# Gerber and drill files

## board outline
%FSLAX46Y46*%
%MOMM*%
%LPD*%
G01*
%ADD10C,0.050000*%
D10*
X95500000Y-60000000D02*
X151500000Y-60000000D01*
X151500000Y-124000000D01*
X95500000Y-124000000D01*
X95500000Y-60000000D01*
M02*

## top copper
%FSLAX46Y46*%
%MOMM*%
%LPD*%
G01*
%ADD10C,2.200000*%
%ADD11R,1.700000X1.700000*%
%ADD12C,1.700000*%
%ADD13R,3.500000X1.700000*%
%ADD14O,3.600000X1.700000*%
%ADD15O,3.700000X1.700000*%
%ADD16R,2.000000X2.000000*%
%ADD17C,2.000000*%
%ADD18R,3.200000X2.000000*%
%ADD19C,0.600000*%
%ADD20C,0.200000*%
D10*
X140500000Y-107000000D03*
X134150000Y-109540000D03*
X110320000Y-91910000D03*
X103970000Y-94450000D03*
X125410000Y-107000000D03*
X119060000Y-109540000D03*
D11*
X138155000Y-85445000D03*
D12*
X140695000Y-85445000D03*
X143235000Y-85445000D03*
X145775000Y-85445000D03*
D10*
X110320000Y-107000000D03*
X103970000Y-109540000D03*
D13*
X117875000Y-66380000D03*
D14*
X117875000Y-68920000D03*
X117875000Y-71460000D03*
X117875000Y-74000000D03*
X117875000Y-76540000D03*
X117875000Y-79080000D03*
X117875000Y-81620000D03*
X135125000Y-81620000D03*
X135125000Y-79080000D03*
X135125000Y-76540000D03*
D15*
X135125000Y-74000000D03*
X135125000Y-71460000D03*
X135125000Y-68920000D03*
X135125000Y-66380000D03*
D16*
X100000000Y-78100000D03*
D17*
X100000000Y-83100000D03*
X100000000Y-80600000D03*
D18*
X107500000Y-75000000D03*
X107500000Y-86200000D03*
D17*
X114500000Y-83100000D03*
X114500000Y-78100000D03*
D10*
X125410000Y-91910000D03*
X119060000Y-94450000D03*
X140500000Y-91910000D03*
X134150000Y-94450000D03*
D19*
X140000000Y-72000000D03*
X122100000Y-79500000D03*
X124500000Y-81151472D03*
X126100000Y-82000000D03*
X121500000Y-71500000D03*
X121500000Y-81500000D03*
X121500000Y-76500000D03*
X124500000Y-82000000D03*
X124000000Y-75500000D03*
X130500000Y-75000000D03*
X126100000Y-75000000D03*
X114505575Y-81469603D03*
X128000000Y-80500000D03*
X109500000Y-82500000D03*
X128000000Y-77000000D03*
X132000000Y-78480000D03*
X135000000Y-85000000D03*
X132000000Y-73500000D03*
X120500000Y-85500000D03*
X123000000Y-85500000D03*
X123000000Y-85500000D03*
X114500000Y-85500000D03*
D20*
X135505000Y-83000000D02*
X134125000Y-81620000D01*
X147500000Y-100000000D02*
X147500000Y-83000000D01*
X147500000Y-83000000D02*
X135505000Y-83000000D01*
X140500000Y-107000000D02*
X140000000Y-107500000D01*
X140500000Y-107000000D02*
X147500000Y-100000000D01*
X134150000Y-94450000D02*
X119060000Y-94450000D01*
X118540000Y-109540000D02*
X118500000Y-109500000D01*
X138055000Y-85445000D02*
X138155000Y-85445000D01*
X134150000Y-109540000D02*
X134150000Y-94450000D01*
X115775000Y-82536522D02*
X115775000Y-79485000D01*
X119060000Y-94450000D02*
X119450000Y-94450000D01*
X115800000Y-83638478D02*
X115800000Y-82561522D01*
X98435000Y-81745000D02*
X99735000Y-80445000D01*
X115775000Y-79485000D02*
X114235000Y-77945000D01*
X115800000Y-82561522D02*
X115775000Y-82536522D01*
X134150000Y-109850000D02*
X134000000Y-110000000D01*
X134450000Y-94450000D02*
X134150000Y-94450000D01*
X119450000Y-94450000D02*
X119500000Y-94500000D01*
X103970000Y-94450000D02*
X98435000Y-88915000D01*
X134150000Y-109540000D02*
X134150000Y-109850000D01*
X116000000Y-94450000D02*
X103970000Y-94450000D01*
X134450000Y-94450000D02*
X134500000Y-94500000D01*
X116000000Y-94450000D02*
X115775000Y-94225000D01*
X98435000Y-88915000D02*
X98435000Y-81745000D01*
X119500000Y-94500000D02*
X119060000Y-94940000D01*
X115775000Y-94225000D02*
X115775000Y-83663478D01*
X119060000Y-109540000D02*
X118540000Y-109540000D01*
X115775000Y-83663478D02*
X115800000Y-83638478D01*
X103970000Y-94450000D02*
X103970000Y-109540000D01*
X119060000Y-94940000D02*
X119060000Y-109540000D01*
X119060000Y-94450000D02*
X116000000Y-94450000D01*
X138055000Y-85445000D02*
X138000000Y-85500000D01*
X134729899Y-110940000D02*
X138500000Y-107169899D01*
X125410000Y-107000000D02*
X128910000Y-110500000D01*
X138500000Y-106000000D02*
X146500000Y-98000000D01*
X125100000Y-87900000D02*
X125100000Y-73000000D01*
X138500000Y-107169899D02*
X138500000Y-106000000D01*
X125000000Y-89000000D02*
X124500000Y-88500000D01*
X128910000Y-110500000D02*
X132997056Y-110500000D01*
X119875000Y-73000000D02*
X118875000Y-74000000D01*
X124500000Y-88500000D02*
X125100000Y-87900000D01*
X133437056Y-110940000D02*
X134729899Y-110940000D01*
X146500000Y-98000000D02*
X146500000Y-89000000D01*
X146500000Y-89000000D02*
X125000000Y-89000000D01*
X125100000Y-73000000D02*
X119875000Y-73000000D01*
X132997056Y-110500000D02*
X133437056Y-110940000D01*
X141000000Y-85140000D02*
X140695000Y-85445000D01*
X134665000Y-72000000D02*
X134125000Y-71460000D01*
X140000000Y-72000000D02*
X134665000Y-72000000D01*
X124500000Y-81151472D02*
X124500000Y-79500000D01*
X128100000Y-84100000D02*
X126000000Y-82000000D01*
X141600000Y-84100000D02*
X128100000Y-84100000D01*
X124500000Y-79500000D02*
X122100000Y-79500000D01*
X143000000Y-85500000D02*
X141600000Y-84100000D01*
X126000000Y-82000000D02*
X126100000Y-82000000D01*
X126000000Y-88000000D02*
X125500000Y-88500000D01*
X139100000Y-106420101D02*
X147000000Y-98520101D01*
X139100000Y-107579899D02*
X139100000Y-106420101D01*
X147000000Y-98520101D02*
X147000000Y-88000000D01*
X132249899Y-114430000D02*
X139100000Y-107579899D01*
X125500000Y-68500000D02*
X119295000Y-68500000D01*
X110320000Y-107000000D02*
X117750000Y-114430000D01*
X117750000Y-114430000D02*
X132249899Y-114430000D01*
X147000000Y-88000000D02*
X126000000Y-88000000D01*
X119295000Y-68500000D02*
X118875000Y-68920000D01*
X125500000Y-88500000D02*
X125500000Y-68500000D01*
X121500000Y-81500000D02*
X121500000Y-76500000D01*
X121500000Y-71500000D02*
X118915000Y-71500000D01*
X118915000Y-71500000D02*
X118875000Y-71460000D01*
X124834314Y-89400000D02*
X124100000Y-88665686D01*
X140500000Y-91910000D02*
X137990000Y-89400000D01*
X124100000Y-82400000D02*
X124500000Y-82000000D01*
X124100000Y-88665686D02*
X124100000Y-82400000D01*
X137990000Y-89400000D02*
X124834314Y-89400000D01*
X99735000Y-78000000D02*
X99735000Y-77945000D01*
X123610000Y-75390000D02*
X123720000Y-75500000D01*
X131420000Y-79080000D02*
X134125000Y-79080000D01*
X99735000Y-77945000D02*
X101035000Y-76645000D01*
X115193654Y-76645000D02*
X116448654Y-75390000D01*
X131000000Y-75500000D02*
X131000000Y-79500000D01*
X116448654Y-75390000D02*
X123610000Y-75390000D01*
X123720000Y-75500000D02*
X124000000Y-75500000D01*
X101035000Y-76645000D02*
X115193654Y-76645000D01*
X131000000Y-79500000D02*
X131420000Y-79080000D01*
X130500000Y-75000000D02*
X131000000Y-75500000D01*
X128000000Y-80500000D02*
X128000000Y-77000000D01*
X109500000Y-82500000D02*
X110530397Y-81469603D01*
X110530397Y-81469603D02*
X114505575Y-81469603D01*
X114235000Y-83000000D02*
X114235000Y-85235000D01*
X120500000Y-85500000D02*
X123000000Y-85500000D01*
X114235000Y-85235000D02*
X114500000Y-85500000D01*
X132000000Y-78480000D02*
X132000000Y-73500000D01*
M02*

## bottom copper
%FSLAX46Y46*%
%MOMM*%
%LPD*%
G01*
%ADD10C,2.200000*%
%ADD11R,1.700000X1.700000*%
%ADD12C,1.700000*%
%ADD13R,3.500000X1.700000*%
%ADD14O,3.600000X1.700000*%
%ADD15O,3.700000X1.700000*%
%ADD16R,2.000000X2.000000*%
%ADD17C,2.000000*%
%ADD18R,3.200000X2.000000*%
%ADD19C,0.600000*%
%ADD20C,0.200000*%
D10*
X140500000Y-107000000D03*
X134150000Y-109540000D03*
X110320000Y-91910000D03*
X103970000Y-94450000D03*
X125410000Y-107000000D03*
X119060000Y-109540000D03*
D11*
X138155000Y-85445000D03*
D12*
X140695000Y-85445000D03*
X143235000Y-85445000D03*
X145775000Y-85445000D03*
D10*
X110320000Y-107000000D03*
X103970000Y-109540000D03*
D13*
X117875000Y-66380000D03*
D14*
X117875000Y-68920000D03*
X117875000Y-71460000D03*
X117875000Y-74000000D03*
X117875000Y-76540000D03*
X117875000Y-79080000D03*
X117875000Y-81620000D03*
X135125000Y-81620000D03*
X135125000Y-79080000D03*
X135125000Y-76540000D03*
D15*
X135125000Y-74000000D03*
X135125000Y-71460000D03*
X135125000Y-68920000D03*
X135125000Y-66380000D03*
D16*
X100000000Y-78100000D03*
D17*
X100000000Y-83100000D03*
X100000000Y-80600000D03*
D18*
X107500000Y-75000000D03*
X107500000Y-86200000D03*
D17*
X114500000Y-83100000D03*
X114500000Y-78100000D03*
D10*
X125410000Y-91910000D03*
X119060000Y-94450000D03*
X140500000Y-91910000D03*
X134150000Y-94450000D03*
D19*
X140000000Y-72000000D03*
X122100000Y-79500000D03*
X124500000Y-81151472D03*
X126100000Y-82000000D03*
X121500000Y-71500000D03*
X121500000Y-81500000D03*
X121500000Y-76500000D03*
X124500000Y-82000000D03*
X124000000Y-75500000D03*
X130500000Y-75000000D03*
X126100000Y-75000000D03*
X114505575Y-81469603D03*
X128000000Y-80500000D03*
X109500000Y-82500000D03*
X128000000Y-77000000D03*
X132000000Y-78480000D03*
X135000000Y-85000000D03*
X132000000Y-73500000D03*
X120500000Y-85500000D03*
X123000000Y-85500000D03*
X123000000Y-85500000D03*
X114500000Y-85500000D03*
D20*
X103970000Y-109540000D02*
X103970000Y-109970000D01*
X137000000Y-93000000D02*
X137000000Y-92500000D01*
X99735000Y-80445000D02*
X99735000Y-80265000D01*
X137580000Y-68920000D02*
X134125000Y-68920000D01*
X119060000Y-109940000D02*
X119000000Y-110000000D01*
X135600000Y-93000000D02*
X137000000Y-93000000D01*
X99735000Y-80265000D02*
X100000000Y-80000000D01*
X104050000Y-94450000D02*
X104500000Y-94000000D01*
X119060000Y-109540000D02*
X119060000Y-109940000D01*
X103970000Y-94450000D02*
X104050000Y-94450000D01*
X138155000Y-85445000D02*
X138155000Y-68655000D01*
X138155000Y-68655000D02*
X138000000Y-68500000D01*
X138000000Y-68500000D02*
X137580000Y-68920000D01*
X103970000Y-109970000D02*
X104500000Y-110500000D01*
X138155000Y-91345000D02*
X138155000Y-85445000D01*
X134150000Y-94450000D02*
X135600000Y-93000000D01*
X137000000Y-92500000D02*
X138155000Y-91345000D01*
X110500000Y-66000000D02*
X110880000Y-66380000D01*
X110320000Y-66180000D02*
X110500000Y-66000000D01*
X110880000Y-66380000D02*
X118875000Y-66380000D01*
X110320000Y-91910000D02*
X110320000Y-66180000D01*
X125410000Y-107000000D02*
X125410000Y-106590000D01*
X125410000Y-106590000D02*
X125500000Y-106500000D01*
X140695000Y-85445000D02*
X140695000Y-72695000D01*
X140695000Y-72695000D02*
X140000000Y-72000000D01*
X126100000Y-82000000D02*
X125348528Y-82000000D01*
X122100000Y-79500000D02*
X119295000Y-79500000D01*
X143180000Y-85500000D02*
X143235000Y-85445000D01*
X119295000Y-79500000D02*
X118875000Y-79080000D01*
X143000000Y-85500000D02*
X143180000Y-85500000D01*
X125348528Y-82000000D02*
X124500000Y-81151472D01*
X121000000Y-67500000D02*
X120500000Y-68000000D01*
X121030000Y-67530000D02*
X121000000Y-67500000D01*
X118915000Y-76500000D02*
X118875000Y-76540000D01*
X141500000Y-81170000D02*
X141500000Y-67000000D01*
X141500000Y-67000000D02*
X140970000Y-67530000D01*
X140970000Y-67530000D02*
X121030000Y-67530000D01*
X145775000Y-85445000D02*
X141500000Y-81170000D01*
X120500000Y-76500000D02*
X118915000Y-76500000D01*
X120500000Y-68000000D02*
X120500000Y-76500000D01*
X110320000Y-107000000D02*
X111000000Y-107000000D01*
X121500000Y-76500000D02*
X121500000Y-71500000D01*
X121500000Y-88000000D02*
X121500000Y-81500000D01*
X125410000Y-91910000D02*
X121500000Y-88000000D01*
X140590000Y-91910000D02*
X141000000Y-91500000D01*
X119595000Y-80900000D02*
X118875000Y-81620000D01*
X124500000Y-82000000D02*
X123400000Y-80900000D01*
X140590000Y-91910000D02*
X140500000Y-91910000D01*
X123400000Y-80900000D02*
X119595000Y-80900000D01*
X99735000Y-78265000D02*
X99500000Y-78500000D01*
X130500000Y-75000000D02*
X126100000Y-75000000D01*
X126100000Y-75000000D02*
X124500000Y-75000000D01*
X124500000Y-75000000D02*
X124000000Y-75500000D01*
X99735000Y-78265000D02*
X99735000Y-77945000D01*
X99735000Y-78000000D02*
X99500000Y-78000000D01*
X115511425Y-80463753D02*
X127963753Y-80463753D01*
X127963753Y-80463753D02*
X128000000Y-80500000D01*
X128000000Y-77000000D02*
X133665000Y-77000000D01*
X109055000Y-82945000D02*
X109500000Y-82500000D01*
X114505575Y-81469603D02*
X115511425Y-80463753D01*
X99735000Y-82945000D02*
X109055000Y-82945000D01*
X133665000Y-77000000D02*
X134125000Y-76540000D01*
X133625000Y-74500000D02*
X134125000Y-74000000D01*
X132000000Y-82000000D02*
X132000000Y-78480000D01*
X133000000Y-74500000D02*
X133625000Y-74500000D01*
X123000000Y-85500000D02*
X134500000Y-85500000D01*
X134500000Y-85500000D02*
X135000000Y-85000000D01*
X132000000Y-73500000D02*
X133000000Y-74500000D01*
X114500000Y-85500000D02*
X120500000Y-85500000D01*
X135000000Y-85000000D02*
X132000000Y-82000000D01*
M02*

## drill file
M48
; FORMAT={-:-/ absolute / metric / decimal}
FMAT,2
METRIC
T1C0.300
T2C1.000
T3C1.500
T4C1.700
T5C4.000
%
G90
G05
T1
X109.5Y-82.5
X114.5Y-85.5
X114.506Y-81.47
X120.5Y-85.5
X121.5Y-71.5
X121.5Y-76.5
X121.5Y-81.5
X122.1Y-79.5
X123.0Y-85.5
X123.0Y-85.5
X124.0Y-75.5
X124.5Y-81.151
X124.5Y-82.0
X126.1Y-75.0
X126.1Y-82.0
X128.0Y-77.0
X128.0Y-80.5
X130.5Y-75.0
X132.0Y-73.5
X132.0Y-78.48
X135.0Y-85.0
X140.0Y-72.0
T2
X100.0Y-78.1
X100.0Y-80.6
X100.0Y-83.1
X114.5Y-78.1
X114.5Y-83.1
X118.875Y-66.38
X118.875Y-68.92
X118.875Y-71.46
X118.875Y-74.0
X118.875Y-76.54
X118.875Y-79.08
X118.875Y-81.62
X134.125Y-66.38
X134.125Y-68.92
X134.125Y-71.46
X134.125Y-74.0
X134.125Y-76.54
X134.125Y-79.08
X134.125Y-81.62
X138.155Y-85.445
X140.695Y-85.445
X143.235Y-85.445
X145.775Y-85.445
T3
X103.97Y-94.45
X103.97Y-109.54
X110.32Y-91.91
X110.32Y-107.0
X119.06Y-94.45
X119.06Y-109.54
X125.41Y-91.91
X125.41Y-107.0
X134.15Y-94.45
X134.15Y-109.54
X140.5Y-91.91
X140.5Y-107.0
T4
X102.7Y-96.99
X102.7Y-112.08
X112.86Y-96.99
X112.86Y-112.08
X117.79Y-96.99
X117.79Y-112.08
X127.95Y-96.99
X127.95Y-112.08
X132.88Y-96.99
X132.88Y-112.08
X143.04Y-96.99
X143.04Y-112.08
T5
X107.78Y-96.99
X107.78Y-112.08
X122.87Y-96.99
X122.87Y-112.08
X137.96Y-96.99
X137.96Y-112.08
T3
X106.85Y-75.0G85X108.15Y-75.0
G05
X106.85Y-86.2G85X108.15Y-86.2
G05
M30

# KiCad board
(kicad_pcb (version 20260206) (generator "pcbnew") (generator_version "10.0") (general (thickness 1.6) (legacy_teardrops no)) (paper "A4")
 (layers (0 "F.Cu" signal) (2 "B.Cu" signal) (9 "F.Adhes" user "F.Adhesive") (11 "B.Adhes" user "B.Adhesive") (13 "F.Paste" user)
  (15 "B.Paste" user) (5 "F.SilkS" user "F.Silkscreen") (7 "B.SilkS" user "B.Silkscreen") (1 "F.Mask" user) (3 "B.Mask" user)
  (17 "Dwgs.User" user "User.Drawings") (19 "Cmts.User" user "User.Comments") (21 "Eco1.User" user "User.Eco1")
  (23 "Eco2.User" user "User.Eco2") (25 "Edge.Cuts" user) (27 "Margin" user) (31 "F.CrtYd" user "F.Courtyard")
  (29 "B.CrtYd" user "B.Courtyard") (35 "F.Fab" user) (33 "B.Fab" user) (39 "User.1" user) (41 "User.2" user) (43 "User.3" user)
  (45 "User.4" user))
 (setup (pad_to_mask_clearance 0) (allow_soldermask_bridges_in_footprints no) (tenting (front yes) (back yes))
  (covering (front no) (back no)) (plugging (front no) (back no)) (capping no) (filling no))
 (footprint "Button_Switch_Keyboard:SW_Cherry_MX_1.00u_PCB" (layer "F.Cu") (at 140.5 107)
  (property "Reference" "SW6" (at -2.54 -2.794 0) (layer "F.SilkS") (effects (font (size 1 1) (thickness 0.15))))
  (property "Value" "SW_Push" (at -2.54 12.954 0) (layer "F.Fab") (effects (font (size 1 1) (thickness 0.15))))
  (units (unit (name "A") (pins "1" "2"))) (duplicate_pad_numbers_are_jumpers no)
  (pad "" np_thru_hole circle (at -7.62 5.08) (size 1.7 1.7) (drill 1.7) (layers "*.Cu" "*.Mask"))
  (pad "" np_thru_hole circle (at -2.54 5.08) (size 4 4) (drill 4) (layers "*.Cu" "*.Mask"))
  (pad "" np_thru_hole circle (at 2.54 5.08) (size 1.7 1.7) (drill 1.7) (layers "*.Cu" "*.Mask"))
  (pad "1" thru_hole circle (at 0 0) (size 2.2 2.2) (drill 1.5) (layers "*.Cu" "*.Mask") (remove_unused_layers no) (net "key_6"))
  (pad "2" thru_hole circle (at -6.35 2.54) (size 2.2 2.2) (drill 1.5) (layers "*.Cu" "*.Mask") (remove_unused_layers no) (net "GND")))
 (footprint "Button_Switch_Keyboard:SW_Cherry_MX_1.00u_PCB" (layer "F.Cu") (at 110.32 91.91)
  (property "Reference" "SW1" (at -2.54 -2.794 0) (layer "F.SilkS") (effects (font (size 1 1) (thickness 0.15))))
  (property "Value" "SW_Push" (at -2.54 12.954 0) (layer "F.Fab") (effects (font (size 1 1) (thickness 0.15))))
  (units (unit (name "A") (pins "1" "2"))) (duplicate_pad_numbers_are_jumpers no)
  (pad "" np_thru_hole circle (at -7.62 5.08) (size 1.7 1.7) (drill 1.7) (layers "*.Cu" "*.Mask"))
  (pad "" np_thru_hole circle (at -2.54 5.08) (size 4 4) (drill 4) (layers "*.Cu" "*.Mask"))
  (pad "" np_thru_hole circle (at 2.54 5.08) (size 1.7 1.7) (drill 1.7) (layers "*.Cu" "*.Mask"))
  (pad "1" thru_hole circle (at 0 0) (size 2.2 2.2) (drill 1.5) (layers "*.Cu" "*.Mask") (remove_unused_layers no) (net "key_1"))
  (pad "2" thru_hole circle (at -6.35 2.54) (size 2.2 2.2) (drill 1.5) (layers "*.Cu" "*.Mask") (remove_unused_layers no) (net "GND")))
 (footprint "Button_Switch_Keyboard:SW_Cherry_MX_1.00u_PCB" (layer "F.Cu") (at 125.41 107)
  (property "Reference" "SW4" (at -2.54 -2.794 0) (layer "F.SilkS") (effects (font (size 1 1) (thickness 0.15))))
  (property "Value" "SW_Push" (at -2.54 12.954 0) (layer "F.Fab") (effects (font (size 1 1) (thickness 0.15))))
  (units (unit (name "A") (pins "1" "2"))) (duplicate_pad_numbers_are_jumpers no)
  (pad "" np_thru_hole circle (at -7.62 5.08) (size 1.7 1.7) (drill 1.7) (layers "*.Cu" "*.Mask"))
  (pad "" np_thru_hole circle (at -2.54 5.08) (size 4 4) (drill 4) (layers "*.Cu" "*.Mask"))
  (pad "" np_thru_hole circle (at 2.54 5.08) (size 1.7 1.7) (drill 1.7) (layers "*.Cu" "*.Mask"))
  (pad "1" thru_hole circle (at 0 0) (size 2.2 2.2) (drill 1.5) (layers "*.Cu" "*.Mask") (remove_unused_layers no) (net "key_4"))
  (pad "2" thru_hole circle (at -6.35 2.54) (size 2.2 2.2) (drill 1.5) (layers "*.Cu" "*.Mask") (remove_unused_layers no) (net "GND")))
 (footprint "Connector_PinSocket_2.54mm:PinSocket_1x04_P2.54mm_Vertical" (layer "F.Cu") (at 138.155 85.445 90)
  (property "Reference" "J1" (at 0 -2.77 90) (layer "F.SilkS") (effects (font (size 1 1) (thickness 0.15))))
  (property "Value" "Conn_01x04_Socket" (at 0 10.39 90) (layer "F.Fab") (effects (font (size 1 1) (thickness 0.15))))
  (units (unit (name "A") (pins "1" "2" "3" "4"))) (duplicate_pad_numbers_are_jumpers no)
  (pad "1" thru_hole rect (at 0 0 90) (size 1.7 1.7) (drill 1) (layers "*.Cu" "*.Mask") (remove_unused_layers no) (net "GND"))
  (pad "2" thru_hole circle (at 0 2.54 90) (size 1.7 1.7) (drill 1) (layers "*.Cu" "*.Mask") (remove_unused_layers no) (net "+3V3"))
  (pad "3" thru_hole circle (at 0 5.08 90) (size 1.7 1.7) (drill 1) (layers "*.Cu" "*.Mask") (remove_unused_layers no) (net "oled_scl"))
  (pad "4" thru_hole circle (at 0 7.62 90) (size 1.7 1.7) (drill 1) (layers "*.Cu" "*.Mask") (remove_unused_layers no) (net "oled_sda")))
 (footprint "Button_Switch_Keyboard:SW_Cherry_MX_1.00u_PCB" (layer "F.Cu") (at 110.32 107)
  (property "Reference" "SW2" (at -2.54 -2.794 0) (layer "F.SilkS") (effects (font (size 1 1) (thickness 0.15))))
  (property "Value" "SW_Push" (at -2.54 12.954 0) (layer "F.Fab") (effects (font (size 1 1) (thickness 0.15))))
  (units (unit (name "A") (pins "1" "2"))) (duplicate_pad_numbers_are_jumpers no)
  (pad "" np_thru_hole circle (at -7.62 5.08) (size 1.7 1.7) (drill 1.7) (layers "*.Cu" "*.Mask"))
  (pad "" np_thru_hole circle (at -2.54 5.08) (size 4 4) (drill 4) (layers "*.Cu" "*.Mask"))
  (pad "" np_thru_hole circle (at 2.54 5.08) (size 1.7 1.7) (drill 1.7) (layers "*.Cu" "*.Mask"))
  (pad "1" thru_hole circle (at 0 0) (size 2.2 2.2) (drill 1.5) (layers "*.Cu" "*.Mask") (remove_unused_layers no) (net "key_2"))
  (pad "2" thru_hole circle (at -6.35 2.54) (size 2.2 2.2) (drill 1.5) (layers "*.Cu" "*.Mask") (remove_unused_layers no) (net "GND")))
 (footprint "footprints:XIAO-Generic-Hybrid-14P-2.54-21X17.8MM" (layer "F.Cu") (at 126.5 74)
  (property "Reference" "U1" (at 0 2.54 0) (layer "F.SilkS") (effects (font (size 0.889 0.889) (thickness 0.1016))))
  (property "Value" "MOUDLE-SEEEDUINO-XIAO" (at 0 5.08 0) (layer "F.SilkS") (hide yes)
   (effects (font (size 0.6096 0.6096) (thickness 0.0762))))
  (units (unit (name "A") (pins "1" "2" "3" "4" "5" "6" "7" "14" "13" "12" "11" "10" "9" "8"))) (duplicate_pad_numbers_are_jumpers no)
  (pad "1" thru_hole rect (at -7.625 -7.62) (size 3.5 1.7) (drill 1 (offset -1 0)) (layers "*.Cu" "*.Mask") (remove_unused_layers no)
   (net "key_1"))
  (pad "2" thru_hole oval (at -7.625 -5.08) (size 3.6 1.7) (drill 1 (offset -1 0)) (layers "*.Cu" "*.Mask") (remove_unused_layers no)
   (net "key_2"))
  (pad "3" thru_hole oval (at -7.625 -2.54) (size 3.6 1.7) (drill 1 (offset -1 0)) (layers "*.Cu" "*.Mask") (remove_unused_layers no)
   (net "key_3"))
  (pad "4" thru_hole oval (at -7.625 0) (size 3.6 1.7) (drill 1 (offset -1 0)) (layers "*.Cu" "*.Mask") (remove_unused_layers no)
   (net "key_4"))
  (pad "5" thru_hole oval (at -7.625 2.54) (size 3.6 1.7) (drill 1 (offset -1 0)) (layers "*.Cu" "*.Mask") (remove_unused_layers no)
   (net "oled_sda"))
  (pad "6" thru_hole oval (at -7.625 5.08 180) (size 3.6 1.7) (drill 1 (offset 1 0)) (layers "*.Cu" "*.Mask") (remove_unused_layers no)
   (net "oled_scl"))
  (pad "7" thru_hole oval (at -7.625 7.62) (size 3.6 1.7) (drill 1 (offset -1 0)) (layers "*.Cu" "*.Mask") (remove_unused_layers no)
   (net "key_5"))
  (pad "8" thru_hole oval (at 7.625 7.62) (size 3.6 1.7) (drill 1 (offset 1 0)) (layers "*.Cu" "*.Mask") (remove_unused_layers no)
   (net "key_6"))
  (pad "9" thru_hole oval (at 7.625 5.08) (size 3.6 1.7) (drill 1 (offset 1 0)) (layers "*.Cu" "*.Mask") (remove_unused_layers no)
   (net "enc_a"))
  (pad "10" thru_hole oval (at 7.625 2.54) (size 3.6 1.7) (drill 1 (offset 1 0)) (layers "*.Cu" "*.Mask") (remove_unused_layers no)
   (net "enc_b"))
  (pad "11" thru_hole oval (at 7.625 0) (size 3.7 1.7) (drill 1 (offset 1 0)) (layers "*.Cu" "*.Mask") (remove_unused_layers no)
   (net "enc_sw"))
  (pad "12" thru_hole oval (at 7.625 -2.54) (size 3.7 1.7) (drill 1 (offset 1 0)) (layers "*.Cu" "*.Mask") (remove_unused_layers no)
   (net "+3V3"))
  (pad "13" thru_hole oval (at 7.625 -5.08) (size 3.7 1.7) (drill 1 (offset 1 0)) (layers "*.Cu" "*.Mask") (remove_unused_layers no)
   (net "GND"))
  (pad "14" thru_hole oval (at 7.625 -7.62) (size 3.7 1.7) (drill 1 (offset 1 0)) (layers "*.Cu" "*.Mask") (remove_unused_layers no)
   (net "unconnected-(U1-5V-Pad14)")))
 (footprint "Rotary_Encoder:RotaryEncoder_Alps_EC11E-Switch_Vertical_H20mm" (layer "F.Cu") (at 100 78.1)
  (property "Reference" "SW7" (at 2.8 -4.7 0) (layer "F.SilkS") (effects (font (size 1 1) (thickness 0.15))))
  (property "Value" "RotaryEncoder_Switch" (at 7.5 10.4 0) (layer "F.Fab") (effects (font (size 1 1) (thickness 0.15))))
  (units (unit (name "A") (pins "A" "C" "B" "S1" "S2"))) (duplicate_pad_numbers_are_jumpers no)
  (pad "A" thru_hole rect (at 0 0) (size 2 2) (drill 1) (layers "*.Cu" "*.Mask") (remove_unused_layers no) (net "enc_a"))
  (pad "B" thru_hole circle (at 0 5) (size 2 2) (drill 1) (layers "*.Cu" "*.Mask") (remove_unused_layers no) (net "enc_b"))
  (pad "C" thru_hole circle (at 0 2.5) (size 2 2) (drill 1) (layers "*.Cu" "*.Mask") (remove_unused_layers no) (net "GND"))
  (pad "MP" thru_hole rect (at 7.5 -3.1) (size 3.2 2) (drill oval 2.8 1.5) (layers "*.Cu" "*.Mask") (remove_unused_layers no))
  (pad "MP" thru_hole rect (at 7.5 8.1) (size 3.2 2) (drill oval 2.8 1.5) (layers "*.Cu" "*.Mask") (remove_unused_layers no))
  (pad "S1" thru_hole circle (at 14.5 5) (size 2 2) (drill 1) (layers "*.Cu" "*.Mask") (remove_unused_layers no) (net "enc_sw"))
  (pad "S2" thru_hole circle (at 14.5 0) (size 2 2) (drill 1) (layers "*.Cu" "*.Mask") (remove_unused_layers no) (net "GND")))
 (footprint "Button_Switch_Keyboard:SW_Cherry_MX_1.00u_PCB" (layer "F.Cu") (at 125.41 91.91)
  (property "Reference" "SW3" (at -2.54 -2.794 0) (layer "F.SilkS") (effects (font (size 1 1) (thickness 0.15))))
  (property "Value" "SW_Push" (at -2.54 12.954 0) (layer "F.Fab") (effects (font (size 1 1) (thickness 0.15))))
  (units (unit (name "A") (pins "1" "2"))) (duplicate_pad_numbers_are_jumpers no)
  (pad "" np_thru_hole circle (at -7.62 5.08) (size 1.7 1.7) (drill 1.7) (layers "*.Cu" "*.Mask"))
  (pad "" np_thru_hole circle (at -2.54 5.08) (size 4 4) (drill 4) (layers "*.Cu" "*.Mask"))
  (pad "" np_thru_hole circle (at 2.54 5.08) (size 1.7 1.7) (drill 1.7) (layers "*.Cu" "*.Mask"))
  (pad "1" thru_hole circle (at 0 0) (size 2.2 2.2) (drill 1.5) (layers "*.Cu" "*.Mask") (remove_unused_layers no) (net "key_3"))
  (pad "2" thru_hole circle (at -6.35 2.54) (size 2.2 2.2) (drill 1.5) (layers "*.Cu" "*.Mask") (remove_unused_layers no) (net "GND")))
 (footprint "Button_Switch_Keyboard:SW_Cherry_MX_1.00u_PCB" (layer "F.Cu") (at 140.5 91.91)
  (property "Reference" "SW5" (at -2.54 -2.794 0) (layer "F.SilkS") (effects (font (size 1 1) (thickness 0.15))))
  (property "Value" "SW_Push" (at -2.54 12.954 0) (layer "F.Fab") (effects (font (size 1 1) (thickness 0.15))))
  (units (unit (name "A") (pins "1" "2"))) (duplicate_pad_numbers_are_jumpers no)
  (pad "" np_thru_hole circle (at -7.62 5.08) (size 1.7 1.7) (drill 1.7) (layers "*.Cu" "*.Mask"))
  (pad "" np_thru_hole circle (at -2.54 5.08) (size 4 4) (drill 4) (layers "*.Cu" "*.Mask"))
  (pad "" np_thru_hole circle (at 2.54 5.08) (size 1.7 1.7) (drill 1.7) (layers "*.Cu" "*.Mask"))
  (pad "1" thru_hole circle (at 0 0) (size 2.2 2.2) (drill 1.5) (layers "*.Cu" "*.Mask") (remove_unused_layers no) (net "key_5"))
  (pad "2" thru_hole circle (at -6.35 2.54) (size 2.2 2.2) (drill 1.5) (layers "*.Cu" "*.Mask") (remove_unused_layers no) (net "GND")))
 (gr_rect (start 95.5 60) (end 151.5 124) (stroke (width 0.05) (type default)) (fill no) (layer "Edge.Cuts"))
 (segment (start 135.505 83) (end 134.125 81.62) (width 0.2) (layer "F.Cu") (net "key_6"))
 (segment (start 147.5 100) (end 147.5 83) (width 0.2) (layer "F.Cu") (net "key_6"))
 (segment (start 147.5 83) (end 135.505 83) (width 0.2) (layer "F.Cu") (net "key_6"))
 (segment (start 140.5 107) (end 140 107.5) (width 0.2) (layer "F.Cu") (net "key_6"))
 (segment (start 140.5 107) (end 147.5 100) (width 0.2) (layer "F.Cu") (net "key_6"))
 (segment (start 134.15 94.45) (end 119.06 94.45) (width 0.2) (layer "F.Cu") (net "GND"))
 (segment (start 118.54 109.54) (end 118.5 109.5) (width 0.2) (layer "F.Cu") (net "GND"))
 (segment (start 138.055 85.445) (end 138.155 85.445) (width 0.2) (layer "F.Cu") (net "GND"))
 (segment (start 134.15 109.54) (end 134.15 94.45) (width 0.2) (layer "F.Cu") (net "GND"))
 (segment (start 115.775 82.536522) (end 115.775 79.485) (width 0.2) (layer "F.Cu") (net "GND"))
 (segment (start 119.06 94.45) (end 119.45 94.45) (width 0.2) (layer "F.Cu") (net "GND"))
 (segment (start 115.8 83.638478) (end 115.8 82.561522) (width 0.2) (layer "F.Cu") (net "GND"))
 (segment (start 98.435 81.745) (end 99.735 80.445) (width 0.2) (layer "F.Cu") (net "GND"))
 (segment (start 115.775 79.485) (end 114.235 77.945) (width 0.2) (layer "F.Cu") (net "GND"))
 (segment (start 115.8 82.561522) (end 115.775 82.536522) (width 0.2) (layer "F.Cu") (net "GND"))
 (segment (start 134.15 109.85) (end 134 110) (width 0.2) (layer "F.Cu") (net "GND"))
 (segment (start 134.45 94.45) (end 134.15 94.45) (width 0.2) (layer "F.Cu") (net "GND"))
 (segment (start 119.45 94.45) (end 119.5 94.5) (width 0.2) (layer "F.Cu") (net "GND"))
 (segment (start 103.97 94.45) (end 98.435 88.915) (width 0.2) (layer "F.Cu") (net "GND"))
 (segment (start 134.15 109.54) (end 134.15 109.85) (width 0.2) (layer "F.Cu") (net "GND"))
 (segment (start 116 94.45) (end 103.97 94.45) (width 0.2) (layer "F.Cu") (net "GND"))
 (segment (start 134.45 94.45) (end 134.5 94.5) (width 0.2) (layer "F.Cu") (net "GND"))
 (segment (start 116 94.45) (end 115.775 94.225) (width 0.2) (layer "F.Cu") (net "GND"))
 (segment (start 98.435 88.915) (end 98.435 81.745) (width 0.2) (layer "F.Cu") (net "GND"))
 (segment (start 119.5 94.5) (end 119.06 94.94) (width 0.2) (layer "F.Cu") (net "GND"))
 (segment (start 115.775 94.225) (end 115.775 83.663478) (width 0.2) (layer "F.Cu") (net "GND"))
 (segment (start 119.06 109.54) (end 118.54 109.54) (width 0.2) (layer "F.Cu") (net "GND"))
 (segment (start 115.775 83.663478) (end 115.8 83.638478) (width 0.2) (layer "F.Cu") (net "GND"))
 (segment (start 103.97 94.45) (end 103.97 109.54) (width 0.2) (layer "F.Cu") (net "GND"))
 (segment (start 119.06 94.94) (end 119.06 109.54) (width 0.2) (layer "F.Cu") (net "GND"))
 (segment (start 119.06 94.45) (end 116 94.45) (width 0.2) (layer "F.Cu") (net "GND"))
 (segment (start 138.055 85.445) (end 138 85.5) (width 0.2) (layer "F.Cu") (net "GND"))
 (segment (start 103.97 109.54) (end 103.97 109.97) (width 0.2) (layer "B.Cu") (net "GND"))
 (segment (start 137 93) (end 137 92.5) (width 0.2) (layer "B.Cu") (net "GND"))
 (segment (start 99.735 80.445) (end 99.735 80.265) (width 0.2) (layer "B.Cu") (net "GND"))
 (segment (start 137.58 68.92) (end 134.125 68.92) (width 0.2) (layer "B.Cu") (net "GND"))
 (segment (start 119.06 109.94) (end 119 110) (width 0.2) (layer "B.Cu") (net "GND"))
 (segment (start 135.6 93) (end 137 93) (width 0.2) (layer "B.Cu") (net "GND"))
 (segment (start 99.735 80.265) (end 100 80) (width 0.2) (layer "B.Cu") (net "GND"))
 (segment (start 104.05 94.45) (end 104.5 94) (width 0.2) (layer "B.Cu") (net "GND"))
 (segment (start 119.06 109.54) (end 119.06 109.94) (width 0.2) (layer "B.Cu") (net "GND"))
 (segment (start 103.97 94.45) (end 104.05 94.45) (width 0.2) (layer "B.Cu") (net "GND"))
 (segment (start 138.155 85.445) (end 138.155 68.655) (width 0.2) (layer "B.Cu") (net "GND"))
 (segment (start 138.155 68.655) (end 138 68.5) (width 0.2) (layer "B.Cu") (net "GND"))
 (segment (start 138 68.5) (end 137.58 68.92) (width 0.2) (layer "B.Cu") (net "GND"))
 (segment (start 103.97 109.97) (end 104.5 110.5) (width 0.2) (layer "B.Cu") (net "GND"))
 (segment (start 138.155 91.345) (end 138.155 85.445) (width 0.2) (layer "B.Cu") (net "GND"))
 (segment (start 134.15 94.45) (end 135.6 93) (width 0.2) (layer "B.Cu") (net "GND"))
 (segment (start 137 92.5) (end 138.155 91.345) (width 0.2) (layer "B.Cu") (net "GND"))
 (segment (start 110.5 66) (end 110.88 66.38) (width 0.2) (layer "B.Cu") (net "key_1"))
 (segment (start 110.32 66.18) (end 110.5 66) (width 0.2) (layer "B.Cu") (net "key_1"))
 (segment (start 110.88 66.38) (end 118.875 66.38) (width 0.2) (layer "B.Cu") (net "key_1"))
 (segment (start 110.32 91.91) (end 110.32 66.18) (width 0.2) (layer "B.Cu") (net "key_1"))
 (segment (start 134.729899 110.94) (end 138.5 107.169899) (width 0.2) (layer "F.Cu") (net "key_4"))
 (segment (start 125.41 107) (end 128.91 110.5) (width 0.2) (layer "F.Cu") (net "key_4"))
 (segment (start 138.5 106) (end 146.5 98) (width 0.2) (layer "F.Cu") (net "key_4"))
 (segment (start 125.1 87.9) (end 125.1 73) (width 0.2) (layer "F.Cu") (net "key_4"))
 (segment (start 138.5 107.169899) (end 138.5 106) (width 0.2) (layer "F.Cu") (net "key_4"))
 (segment (start 125 89) (end 124.5 88.5) (width 0.2) (layer "F.Cu") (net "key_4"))
 (segment (start 128.91 110.5) (end 132.997056 110.5) (width 0.2) (layer "F.Cu") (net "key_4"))
 (segment (start 119.875 73) (end 118.875 74) (width 0.2) (layer "F.Cu") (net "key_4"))
 (segment (start 124.5 88.5) (end 125.1 87.9) (width 0.2) (layer "F.Cu") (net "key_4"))
 (segment (start 133.437056 110.94) (end 134.729899 110.94) (width 0.2) (layer "F.Cu") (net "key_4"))
 (segment (start 146.5 98) (end 146.5 89) (width 0.2) (layer "F.Cu") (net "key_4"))
 (segment (start 146.5 89) (end 125 89) (width 0.2) (layer "F.Cu") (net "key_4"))
 (segment (start 125.1 73) (end 119.875 73) (width 0.2) (layer "F.Cu") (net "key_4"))
 (segment (start 132.997056 110.5) (end 133.437056 110.94) (width 0.2) (layer "F.Cu") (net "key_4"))
 (segment (start 125.41 107) (end 125.41 106.59) (width 0.2) (layer "B.Cu") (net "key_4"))
 (segment (start 125.41 106.59) (end 125.5 106.5) (width 0.2) (layer "B.Cu") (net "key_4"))
 (segment (start 141 85.14) (end 140.695 85.445) (width 0.2) (layer "F.Cu") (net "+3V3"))
 (segment (start 134.665 72) (end 134.125 71.46) (width 0.2) (layer "F.Cu") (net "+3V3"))
 (segment (start 140 72) (end 134.665 72) (width 0.2) (layer "F.Cu") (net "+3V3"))
 (via (at 140 72) (size 0.6) (drill 0.3) (layers "F.Cu" "B.Cu") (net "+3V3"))
 (segment (start 140.695 85.445) (end 140.695 72.695) (width 0.2) (layer "B.Cu") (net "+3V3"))
 (segment (start 140.695 72.695) (end 140 72) (width 0.2) (layer "B.Cu") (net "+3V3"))
 (segment (start 124.5 81.151472) (end 124.5 79.5) (width 0.2) (layer "F.Cu") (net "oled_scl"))
 (segment (start 128.1 84.1) (end 126 82) (width 0.2) (layer "F.Cu") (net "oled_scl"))
 (segment (start 141.6 84.1) (end 128.1 84.1) (width 0.2) (layer "F.Cu") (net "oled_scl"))
 (segment (start 124.5 79.5) (end 122.1 79.5) (width 0.2) (layer "F.Cu") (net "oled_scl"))
 (segment (start 143 85.5) (end 141.6 84.1) (width 0.2) (layer "F.Cu") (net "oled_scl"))
 (segment (start 126 82) (end 126.1 82) (width 0.2) (layer "F.Cu") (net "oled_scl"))
 (via (at 122.1 79.5) (size 0.6) (drill 0.3) (layers "F.Cu" "B.Cu") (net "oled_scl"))
 (via (at 124.5 81.151472) (size 0.6) (drill 0.3) (layers "F.Cu" "B.Cu") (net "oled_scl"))
 (via (at 126.1 82) (size 0.6) (drill 0.3) (layers "F.Cu" "B.Cu") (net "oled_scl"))
 (segment (start 126.1 82) (end 125.348528 82) (width 0.2) (layer "B.Cu") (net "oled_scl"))
 (segment (start 122.1 79.5) (end 119.295 79.5) (width 0.2) (layer "B.Cu") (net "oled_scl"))
 (segment (start 143.18 85.5) (end 143.235 85.445) (width 0.2) (layer "B.Cu") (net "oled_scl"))
 (segment (start 119.295 79.5) (end 118.875 79.08) (width 0.2) (layer "B.Cu") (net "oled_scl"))
 (segment (start 143 85.5) (end 143.18 85.5) (width 0.2) (layer "B.Cu") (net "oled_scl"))
 (segment (start 125.348528 82) (end 124.5 81.151472) (width 0.2) (layer "B.Cu") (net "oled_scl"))
 (segment (start 121 67.5) (end 120.5 68) (width 0.2) (layer "B.Cu") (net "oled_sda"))
 (segment (start 121.03 67.53) (end 121 67.5) (width 0.2) (layer "B.Cu") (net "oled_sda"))
 (segment (start 118.915 76.5) (end 118.875 76.54) (width 0.2) (layer "B.Cu") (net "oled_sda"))
 (segment (start 141.5 81.17) (end 141.5 67) (width 0.2) (layer "B.Cu") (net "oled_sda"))
 (segment (start 141.5 67) (end 140.97 67.53) (width 0.2) (layer "B.Cu") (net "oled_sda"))
 (segment (start 140.97 67.53) (end 121.03 67.53) (width 0.2) (layer "B.Cu") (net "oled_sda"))
 (segment (start 145.775 85.445) (end 141.5 81.17) (width 0.2) (layer "B.Cu") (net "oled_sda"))
 (segment (start 120.5 76.5) (end 118.915 76.5) (width 0.2) (layer "B.Cu") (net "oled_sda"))
 (segment (start 120.5 68) (end 120.5 76.5) (width 0.2) (layer "B.Cu") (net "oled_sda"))
 (segment (start 126 88) (end 125.5 88.5) (width 0.2) (layer "F.Cu") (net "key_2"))
 (segment (start 139.1 106.420101) (end 147 98.520101) (width 0.2) (layer "F.Cu") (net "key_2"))
 (segment (start 139.1 107.579899) (end 139.1 106.420101) (width 0.2) (layer "F.Cu") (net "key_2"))
 (segment (start 147 98.520101) (end 147 88) (width 0.2) (layer "F.Cu") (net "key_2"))
 (segment (start 132.249899 114.43) (end 139.1 107.579899) (width 0.2) (layer "F.Cu") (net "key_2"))
 (segment (start 125.5 68.5) (end 119.295 68.5) (width 0.2) (layer "F.Cu") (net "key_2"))
 (segment (start 110.32 107) (end 117.75 114.43) (width 0.2) (layer "F.Cu") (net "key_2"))
 (segment (start 117.75 114.43) (end 132.249899 114.43) (width 0.2) (layer "F.Cu") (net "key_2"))
 (segment (start 147 88) (end 126 88) (width 0.2) (layer "F.Cu") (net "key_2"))
 (segment (start 119.295 68.5) (end 118.875 68.92) (width 0.2) (layer "F.Cu") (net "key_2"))
 (segment (start 125.5 88.5) (end 125.5 68.5) (width 0.2) (layer "F.Cu") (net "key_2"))
 (segment (start 110.32 107) (end 111 107) (width 0.2) (layer "B.Cu") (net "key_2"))
 (segment (start 121.5 81.5) (end 121.5 76.5) (width 0.2) (layer "F.Cu") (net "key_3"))
 (segment (start 121.5 71.5) (end 118.915 71.5) (width 0.2) (layer "F.Cu") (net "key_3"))
 (segment (start 118.915 71.5) (end 118.875 71.46) (width 0.2) (layer "F.Cu") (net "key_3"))
 (via (at 121.5 71.5) (size 0.6) (drill 0.3) (layers "F.Cu" "B.Cu") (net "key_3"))
 (via (at 121.5 81.5) (size 0.6) (drill 0.3) (layers "F.Cu" "B.Cu") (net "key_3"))
 (via (at 121.5 76.5) (size 0.6) (drill 0.3) (layers "F.Cu" "B.Cu") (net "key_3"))
 (segment (start 121.5 76.5) (end 121.5 71.5) (width 0.2) (layer "B.Cu") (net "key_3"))
 (segment (start 121.5 88) (end 121.5 81.5) (width 0.2) (layer "B.Cu") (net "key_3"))
 (segment (start 125.41 91.91) (end 121.5 88) (width 0.2) (layer "B.Cu") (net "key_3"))
 (segment (start 124.834314 89.4) (end 124.1 88.665686) (width 0.2) (layer "F.Cu") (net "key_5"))
 (segment (start 140.5 91.91) (end 137.99 89.4) (width 0.2) (layer "F.Cu") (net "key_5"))
 (segment (start 124.1 82.4) (end 124.5 82) (width 0.2) (layer "F.Cu") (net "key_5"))
 (segment (start 124.1 88.665686) (end 124.1 82.4) (width 0.2) (layer "F.Cu") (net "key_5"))
 (segment (start 137.99 89.4) (end 124.834314 89.4) (width 0.2) (layer "F.Cu") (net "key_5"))
 (via (at 124.5 82) (size 0.6) (drill 0.3) (layers "F.Cu" "B.Cu") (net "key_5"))
 (segment (start 140.59 91.91) (end 141 91.5) (width 0.2) (layer "B.Cu") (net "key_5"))
 (segment (start 119.595 80.9) (end 118.875 81.62) (width 0.2) (layer "B.Cu") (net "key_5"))
 (segment (start 124.5 82) (end 123.4 80.9) (width 0.2) (layer "B.Cu") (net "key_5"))
 (segment (start 140.59 91.91) (end 140.5 91.91) (width 0.2) (layer "B.Cu") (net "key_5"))
 (segment (start 123.4 80.9) (end 119.595 80.9) (width 0.2) (layer "B.Cu") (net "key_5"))
 (segment (start 99.735 78) (end 99.735 77.945) (width 0.2) (layer "F.Cu") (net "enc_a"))
 (segment (start 123.61 75.39) (end 123.72 75.5) (width 0.2) (layer "F.Cu") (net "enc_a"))
 (segment (start 131.42 79.08) (end 134.125 79.08) (width 0.2) (layer "F.Cu") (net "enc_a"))
 (segment (start 99.735 77.945) (end 101.035 76.645) (width 0.2) (layer "F.Cu") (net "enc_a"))
 (segment (start 115.193654 76.645) (end 116.448654 75.39) (width 0.2) (layer "F.Cu") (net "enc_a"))
 (segment (start 131 75.5) (end 131 79.5) (width 0.2) (layer "F.Cu") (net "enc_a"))
 (segment (start 116.448654 75.39) (end 123.61 75.39) (width 0.2) (layer "F.Cu") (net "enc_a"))
 (segment (start 123.72 75.5) (end 124 75.5) (width 0.2) (layer "F.Cu") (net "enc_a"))
 (segment (start 101.035 76.645) (end 115.193654 76.645) (width 0.2) (layer "F.Cu") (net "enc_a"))
 (segment (start 131 79.5) (end 131.42 79.08) (width 0.2) (layer "F.Cu") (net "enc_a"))
 (segment (start 130.5 75) (end 131 75.5) (width 0.2) (layer "F.Cu") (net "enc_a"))
 (via (at 124 75.5) (size 0.6) (drill 0.3) (layers "F.Cu" "B.Cu") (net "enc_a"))
 (via (at 130.5 75) (size 0.6) (drill 0.3) (layers "F.Cu" "B.Cu") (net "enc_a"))
 (via (at 126.1 75) (size 0.6) (drill 0.3) (layers "F.Cu" "B.Cu") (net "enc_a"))
 (segment (start 99.735 78.265) (end 99.5 78.5) (width 0.2) (layer "B.Cu") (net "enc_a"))
 (segment (start 130.5 75) (end 126.1 75) (width 0.2) (layer "B.Cu") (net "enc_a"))
 (segment (start 126.1 75) (end 124.5 75) (width 0.2) (layer "B.Cu") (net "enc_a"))
 (segment (start 124.5 75) (end 124 75.5) (width 0.2) (layer "B.Cu") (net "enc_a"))
 (segment (start 99.735 78.265) (end 99.735 77.945) (width 0.2) (layer "B.Cu") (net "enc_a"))
 (segment (start 99.735 78) (end 99.5 78) (width 0.2) (layer "B.Cu") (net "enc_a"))
 (segment (start 128 80.5) (end 128 77) (width 0.2) (layer "F.Cu") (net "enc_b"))
 (segment (start 109.5 82.5) (end 110.530397 81.469603) (width 0.2) (layer "F.Cu") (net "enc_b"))
 (segment (start 110.530397 81.469603) (end 114.505575 81.469603) (width 0.2) (layer "F.Cu") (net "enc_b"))
 (via (at 114.505575 81.469603) (size 0.6) (drill 0.3) (layers "F.Cu" "B.Cu") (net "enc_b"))
 (via (at 128 80.5) (size 0.6) (drill 0.3) (layers "F.Cu" "B.Cu") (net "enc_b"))
 (via (at 109.5 82.5) (size 0.6) (drill 0.3) (layers "F.Cu" "B.Cu") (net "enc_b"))
 (via (at 128 77) (size 0.6) (drill 0.3) (layers "F.Cu" "B.Cu") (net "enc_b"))
 (segment (start 115.511425 80.463753) (end 127.963753 80.463753) (width 0.2) (layer "B.Cu") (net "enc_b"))
 (segment (start 127.963753 80.463753) (end 128 80.5) (width 0.2) (layer "B.Cu") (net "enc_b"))
 (segment (start 128 77) (end 133.665 77) (width 0.2) (layer "B.Cu") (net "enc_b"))
 (segment (start 109.055 82.945) (end 109.5 82.5) (width 0.2) (layer "B.Cu") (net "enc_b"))
 (segment (start 114.505575 81.469603) (end 115.511425 80.463753) (width 0.2) (layer "B.Cu") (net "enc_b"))
 (segment (start 99.735 82.945) (end 109.055 82.945) (width 0.2) (layer "B.Cu") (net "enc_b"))
 (segment (start 133.665 77) (end 134.125 76.54) (width 0.2) (layer "B.Cu") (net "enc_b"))
 (segment (start 114.235 83) (end 114.235 85.235) (width 0.2) (layer "F.Cu") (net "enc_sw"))
 (segment (start 120.5 85.5) (end 123 85.5) (width 0.2) (layer "F.Cu") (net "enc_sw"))
 (segment (start 114.235 85.235) (end 114.5 85.5) (width 0.2) (layer "F.Cu") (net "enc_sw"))
 (segment (start 132 78.48) (end 132 73.5) (width 0.2) (layer "F.Cu") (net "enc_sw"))
 (via (at 132 78.48) (size 0.6) (drill 0.3) (layers "F.Cu" "B.Cu") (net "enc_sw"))
 (via (at 135 85) (size 0.6) (drill 0.3) (layers "F.Cu" "B.Cu") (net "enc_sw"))
 (via (at 132 73.5) (size 0.6) (drill 0.3) (layers "F.Cu" "B.Cu") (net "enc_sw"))
 (via (at 120.5 85.5) (size 0.6) (drill 0.3) (layers "F.Cu" "B.Cu") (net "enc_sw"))
 (via (at 123 85.5) (size 0.6) (drill 0.3) (layers "F.Cu" "B.Cu") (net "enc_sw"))
 (via (at 123 85.5) (size 0.6) (drill 0.3) (layers "F.Cu" "B.Cu") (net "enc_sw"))
 (via (at 114.5 85.5) (size 0.6) (drill 0.3) (layers "F.Cu" "B.Cu") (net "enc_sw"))
 (segment (start 133.625 74.5) (end 134.125 74) (width 0.2) (layer "B.Cu") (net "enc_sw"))
 (segment (start 132 82) (end 132 78.48) (width 0.2) (layer "B.Cu") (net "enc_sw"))
 (segment (start 133 74.5) (end 133.625 74.5) (width 0.2) (layer "B.Cu") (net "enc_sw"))
 (segment (start 123 85.5) (end 134.5 85.5) (width 0.2) (layer "B.Cu") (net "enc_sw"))
 (segment (start 134.5 85.5) (end 135 85) (width 0.2) (layer "B.Cu") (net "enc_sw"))
 (segment (start 132 73.5) (end 133 74.5) (width 0.2) (layer "B.Cu") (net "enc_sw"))
 (segment (start 114.5 85.5) (end 120.5 85.5) (width 0.2) (layer "B.Cu") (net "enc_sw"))
 (segment (start 135 85) (end 132 82) (width 0.2) (layer "B.Cu") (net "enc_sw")))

